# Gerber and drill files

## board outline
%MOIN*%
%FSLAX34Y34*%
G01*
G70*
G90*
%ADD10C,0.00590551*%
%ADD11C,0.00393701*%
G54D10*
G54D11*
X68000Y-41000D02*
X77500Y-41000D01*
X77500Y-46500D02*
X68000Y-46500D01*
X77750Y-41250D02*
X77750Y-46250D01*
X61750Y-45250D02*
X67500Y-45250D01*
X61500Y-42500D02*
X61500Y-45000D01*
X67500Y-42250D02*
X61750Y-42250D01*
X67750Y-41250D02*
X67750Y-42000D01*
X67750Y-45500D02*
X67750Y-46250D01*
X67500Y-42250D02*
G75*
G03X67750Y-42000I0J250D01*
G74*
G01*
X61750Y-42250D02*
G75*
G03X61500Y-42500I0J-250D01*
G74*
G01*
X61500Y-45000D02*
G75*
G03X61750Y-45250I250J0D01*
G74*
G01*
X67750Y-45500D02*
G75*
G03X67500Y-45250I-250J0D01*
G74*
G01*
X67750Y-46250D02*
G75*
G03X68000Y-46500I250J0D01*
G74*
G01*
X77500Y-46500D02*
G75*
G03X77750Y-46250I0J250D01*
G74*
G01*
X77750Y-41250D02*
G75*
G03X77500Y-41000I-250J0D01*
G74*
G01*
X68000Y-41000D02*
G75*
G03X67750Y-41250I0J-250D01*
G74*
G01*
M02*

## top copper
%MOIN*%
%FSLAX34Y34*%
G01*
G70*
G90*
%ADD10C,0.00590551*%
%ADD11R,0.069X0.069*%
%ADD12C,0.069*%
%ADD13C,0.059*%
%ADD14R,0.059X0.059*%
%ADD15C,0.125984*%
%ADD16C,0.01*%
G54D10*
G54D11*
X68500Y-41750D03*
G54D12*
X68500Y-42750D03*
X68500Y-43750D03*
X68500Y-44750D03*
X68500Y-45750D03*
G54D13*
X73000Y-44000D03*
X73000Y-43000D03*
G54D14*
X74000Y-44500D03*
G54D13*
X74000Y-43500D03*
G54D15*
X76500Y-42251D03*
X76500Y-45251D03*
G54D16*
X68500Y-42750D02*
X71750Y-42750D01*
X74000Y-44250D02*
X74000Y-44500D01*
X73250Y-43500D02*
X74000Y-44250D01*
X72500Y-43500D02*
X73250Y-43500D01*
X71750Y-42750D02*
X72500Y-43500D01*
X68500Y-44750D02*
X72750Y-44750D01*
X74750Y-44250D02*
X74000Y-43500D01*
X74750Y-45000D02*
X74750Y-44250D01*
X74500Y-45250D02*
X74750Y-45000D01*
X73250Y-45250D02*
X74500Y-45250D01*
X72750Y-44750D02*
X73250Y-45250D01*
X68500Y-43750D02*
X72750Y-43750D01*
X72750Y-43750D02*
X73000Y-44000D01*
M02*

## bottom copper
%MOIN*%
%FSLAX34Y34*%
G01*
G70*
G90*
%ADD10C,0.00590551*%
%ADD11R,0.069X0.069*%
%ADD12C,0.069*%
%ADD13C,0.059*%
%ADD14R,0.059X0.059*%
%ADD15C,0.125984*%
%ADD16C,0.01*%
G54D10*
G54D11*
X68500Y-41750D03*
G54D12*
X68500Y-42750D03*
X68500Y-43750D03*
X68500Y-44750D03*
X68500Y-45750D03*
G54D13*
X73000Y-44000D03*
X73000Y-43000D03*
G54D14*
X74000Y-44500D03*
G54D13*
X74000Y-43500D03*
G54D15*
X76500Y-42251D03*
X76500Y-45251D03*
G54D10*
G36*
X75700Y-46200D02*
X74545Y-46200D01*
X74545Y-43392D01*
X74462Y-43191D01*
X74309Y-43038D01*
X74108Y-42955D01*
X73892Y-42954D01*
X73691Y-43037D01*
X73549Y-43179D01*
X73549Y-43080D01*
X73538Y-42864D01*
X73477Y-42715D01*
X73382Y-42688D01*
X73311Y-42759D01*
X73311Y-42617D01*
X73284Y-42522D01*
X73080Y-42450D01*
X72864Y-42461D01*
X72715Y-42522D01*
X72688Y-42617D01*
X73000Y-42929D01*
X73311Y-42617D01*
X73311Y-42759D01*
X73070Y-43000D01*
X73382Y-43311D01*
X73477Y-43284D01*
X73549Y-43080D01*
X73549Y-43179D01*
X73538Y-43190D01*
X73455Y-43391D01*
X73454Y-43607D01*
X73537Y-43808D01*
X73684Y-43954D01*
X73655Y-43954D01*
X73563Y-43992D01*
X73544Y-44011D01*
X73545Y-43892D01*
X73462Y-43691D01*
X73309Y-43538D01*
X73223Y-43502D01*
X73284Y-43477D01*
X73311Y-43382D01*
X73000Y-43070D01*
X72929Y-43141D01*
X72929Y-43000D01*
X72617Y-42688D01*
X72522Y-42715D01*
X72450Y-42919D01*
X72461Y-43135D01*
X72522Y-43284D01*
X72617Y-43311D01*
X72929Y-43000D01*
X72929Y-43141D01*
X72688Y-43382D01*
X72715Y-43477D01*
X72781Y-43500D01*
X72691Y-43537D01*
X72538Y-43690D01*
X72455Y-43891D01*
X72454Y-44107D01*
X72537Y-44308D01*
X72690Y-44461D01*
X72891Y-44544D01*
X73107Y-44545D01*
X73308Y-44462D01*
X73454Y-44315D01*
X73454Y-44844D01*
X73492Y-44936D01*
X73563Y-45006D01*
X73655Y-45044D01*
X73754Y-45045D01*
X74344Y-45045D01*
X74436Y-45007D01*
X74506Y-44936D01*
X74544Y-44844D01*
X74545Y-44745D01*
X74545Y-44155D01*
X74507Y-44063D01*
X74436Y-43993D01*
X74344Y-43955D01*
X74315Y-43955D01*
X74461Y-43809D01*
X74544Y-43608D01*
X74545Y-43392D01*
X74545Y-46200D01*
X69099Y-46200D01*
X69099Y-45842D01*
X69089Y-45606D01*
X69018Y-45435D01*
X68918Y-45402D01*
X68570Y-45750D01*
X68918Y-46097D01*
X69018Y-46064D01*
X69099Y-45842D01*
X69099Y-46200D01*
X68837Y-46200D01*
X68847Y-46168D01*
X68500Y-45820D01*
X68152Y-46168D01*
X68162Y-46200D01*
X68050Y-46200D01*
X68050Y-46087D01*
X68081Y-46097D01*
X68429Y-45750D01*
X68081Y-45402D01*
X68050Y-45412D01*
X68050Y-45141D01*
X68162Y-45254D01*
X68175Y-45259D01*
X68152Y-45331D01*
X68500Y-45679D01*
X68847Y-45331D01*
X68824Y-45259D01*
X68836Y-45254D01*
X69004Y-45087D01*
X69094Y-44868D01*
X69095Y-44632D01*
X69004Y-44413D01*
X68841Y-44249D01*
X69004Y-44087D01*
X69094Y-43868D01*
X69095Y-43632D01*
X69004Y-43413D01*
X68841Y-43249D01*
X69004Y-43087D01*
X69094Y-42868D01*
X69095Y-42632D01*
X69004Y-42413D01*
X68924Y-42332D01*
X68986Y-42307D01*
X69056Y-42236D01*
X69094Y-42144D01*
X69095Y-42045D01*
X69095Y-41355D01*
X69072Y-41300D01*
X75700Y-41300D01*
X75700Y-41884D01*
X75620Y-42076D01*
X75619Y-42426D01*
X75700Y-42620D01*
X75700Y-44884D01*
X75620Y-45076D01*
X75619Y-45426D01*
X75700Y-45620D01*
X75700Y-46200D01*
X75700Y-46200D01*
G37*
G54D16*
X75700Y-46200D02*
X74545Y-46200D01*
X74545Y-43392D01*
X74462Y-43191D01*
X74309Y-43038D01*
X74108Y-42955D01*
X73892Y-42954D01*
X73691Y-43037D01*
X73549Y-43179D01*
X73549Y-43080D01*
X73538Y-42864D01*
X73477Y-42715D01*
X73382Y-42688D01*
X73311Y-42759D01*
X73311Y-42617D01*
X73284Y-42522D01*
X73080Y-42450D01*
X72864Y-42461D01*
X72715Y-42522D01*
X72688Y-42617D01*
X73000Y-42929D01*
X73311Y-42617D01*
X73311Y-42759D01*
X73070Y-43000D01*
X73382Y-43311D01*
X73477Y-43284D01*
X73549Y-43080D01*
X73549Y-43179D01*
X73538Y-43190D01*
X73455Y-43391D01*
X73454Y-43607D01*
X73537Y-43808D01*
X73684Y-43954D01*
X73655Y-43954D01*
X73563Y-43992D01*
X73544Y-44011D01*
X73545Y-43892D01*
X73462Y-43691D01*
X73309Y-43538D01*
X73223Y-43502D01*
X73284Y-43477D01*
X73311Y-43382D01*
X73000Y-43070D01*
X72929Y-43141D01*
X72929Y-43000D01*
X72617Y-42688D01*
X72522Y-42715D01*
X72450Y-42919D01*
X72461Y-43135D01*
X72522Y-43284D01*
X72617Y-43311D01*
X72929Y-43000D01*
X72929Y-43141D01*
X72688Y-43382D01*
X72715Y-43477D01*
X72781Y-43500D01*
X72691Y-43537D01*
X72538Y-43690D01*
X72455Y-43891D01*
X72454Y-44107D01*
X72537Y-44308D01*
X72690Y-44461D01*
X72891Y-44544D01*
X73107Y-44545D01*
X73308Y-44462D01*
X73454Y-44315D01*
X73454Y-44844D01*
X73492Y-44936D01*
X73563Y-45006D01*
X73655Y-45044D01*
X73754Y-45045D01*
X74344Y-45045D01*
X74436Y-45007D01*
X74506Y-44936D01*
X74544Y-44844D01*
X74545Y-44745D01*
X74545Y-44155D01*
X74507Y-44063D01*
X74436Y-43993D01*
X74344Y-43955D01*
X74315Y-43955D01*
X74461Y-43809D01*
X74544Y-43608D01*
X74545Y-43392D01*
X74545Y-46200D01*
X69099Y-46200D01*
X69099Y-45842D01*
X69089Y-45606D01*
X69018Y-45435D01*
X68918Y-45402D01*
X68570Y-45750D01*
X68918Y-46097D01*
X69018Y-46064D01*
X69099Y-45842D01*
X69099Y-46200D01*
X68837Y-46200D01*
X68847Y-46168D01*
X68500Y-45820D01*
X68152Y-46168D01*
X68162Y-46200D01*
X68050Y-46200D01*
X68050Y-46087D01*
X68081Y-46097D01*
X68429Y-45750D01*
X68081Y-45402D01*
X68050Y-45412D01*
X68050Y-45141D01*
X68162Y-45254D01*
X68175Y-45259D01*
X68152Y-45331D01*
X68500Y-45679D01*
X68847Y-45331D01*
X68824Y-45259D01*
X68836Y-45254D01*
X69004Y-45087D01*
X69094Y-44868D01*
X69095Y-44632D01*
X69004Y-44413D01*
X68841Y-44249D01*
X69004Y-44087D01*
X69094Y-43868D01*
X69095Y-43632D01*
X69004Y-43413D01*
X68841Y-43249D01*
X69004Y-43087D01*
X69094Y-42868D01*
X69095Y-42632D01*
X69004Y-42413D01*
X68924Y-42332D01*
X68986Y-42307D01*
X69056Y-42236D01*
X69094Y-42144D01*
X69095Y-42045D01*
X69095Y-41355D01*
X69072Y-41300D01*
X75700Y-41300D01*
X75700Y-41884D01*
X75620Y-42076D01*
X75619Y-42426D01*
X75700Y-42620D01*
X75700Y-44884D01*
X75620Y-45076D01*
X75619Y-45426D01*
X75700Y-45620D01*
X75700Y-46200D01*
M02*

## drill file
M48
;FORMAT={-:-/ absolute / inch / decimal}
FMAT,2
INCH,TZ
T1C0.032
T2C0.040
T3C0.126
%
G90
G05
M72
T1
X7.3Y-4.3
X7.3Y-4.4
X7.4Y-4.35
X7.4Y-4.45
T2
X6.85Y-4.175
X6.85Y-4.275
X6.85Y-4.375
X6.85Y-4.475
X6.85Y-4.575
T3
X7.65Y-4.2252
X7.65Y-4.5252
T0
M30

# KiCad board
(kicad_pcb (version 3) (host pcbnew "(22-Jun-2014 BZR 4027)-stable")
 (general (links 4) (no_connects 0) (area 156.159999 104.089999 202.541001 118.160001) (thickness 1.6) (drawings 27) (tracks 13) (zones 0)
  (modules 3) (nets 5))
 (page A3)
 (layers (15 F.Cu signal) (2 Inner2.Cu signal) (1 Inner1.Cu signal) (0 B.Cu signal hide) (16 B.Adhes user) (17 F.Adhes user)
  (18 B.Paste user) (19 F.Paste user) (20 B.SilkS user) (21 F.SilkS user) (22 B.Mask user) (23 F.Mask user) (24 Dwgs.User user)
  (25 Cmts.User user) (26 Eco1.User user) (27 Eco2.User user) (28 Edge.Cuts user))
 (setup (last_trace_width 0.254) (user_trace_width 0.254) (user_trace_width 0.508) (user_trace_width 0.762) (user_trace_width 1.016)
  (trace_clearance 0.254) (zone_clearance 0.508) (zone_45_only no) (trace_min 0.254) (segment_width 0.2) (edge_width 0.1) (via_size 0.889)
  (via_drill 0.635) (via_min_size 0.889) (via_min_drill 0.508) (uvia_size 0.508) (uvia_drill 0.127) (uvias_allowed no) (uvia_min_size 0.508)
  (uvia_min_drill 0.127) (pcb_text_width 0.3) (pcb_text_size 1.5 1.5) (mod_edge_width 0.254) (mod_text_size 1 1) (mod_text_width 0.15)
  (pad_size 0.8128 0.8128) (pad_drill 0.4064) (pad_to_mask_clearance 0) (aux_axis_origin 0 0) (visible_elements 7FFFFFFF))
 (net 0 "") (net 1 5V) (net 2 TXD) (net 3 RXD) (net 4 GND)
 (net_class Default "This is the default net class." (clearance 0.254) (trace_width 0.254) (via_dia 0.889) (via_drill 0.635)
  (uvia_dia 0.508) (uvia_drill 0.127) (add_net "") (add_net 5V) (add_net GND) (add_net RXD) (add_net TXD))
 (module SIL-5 (layer F.Cu) (at 173.99 108.585 270)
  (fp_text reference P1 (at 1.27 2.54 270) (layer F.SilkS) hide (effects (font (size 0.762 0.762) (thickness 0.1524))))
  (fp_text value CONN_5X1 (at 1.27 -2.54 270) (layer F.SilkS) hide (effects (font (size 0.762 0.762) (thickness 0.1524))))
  (pad 1 thru_hole rect (at -2.54 0 270) (size 1.7526 1.7526) (drill 1.016) (layers *.Cu *.Mask F.SilkS))
  (pad 2 thru_hole circle (at 0 0 270) (size 1.7526 1.7526) (drill 1.016) (layers *.Cu *.Mask F.SilkS) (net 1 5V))
  (pad 3 thru_hole circle (at 2.54 0 270) (size 1.7526 1.7526) (drill 1.016) (layers *.Cu *.Mask F.SilkS) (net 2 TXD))
  (pad 4 thru_hole circle (at 5.08 0 270) (size 1.7526 1.7526) (drill 1.016) (layers *.Cu *.Mask F.SilkS) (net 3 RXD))
  (pad 5 thru_hole circle (at 7.62 0 270) (size 1.7526 1.7526) (drill 1.016) (layers *.Cu *.Mask F.SilkS) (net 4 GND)))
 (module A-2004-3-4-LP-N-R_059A (layer F.Cu) (at 187.96 113.03 90)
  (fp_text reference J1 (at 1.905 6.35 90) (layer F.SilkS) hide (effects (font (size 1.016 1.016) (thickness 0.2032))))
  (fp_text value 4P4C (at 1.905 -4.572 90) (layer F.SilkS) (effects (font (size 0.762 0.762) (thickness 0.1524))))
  (pad 2 thru_hole circle (at 1.27 -2.54 90) (size 1.4986 1.4986) (drill 0.8128) (layers *.Cu *.Mask F.SilkS) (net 2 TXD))
  (pad 4 thru_hole circle (at 3.81 -2.54 90) (size 1.4986 1.4986) (drill 0.8128) (layers *.Cu *.Mask F.SilkS) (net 4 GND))
  (pad 1 thru_hole rect (at 0 0 90) (size 1.4986 1.4986) (drill 0.8128) (layers *.Cu *.Mask F.SilkS) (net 1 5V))
  (pad 3 thru_hole circle (at 2.54 0 90) (size 1.4986 1.4986) (drill 0.8128) (layers *.Cu *.Mask F.SilkS) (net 3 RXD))
  (pad "" thru_hole circle (at 5.71 6.35 90) (size 3.2 3.2) (drill 3.2) (layers *.Cu *.Mask F.SilkS))
  (pad "" thru_hole circle (at -1.91 6.35 90) (size 3.2 3.2) (drill 3.2) (layers *.Cu *.Mask F.SilkS)))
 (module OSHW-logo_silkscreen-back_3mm (layer F.Cu) (at 169.545 111.125)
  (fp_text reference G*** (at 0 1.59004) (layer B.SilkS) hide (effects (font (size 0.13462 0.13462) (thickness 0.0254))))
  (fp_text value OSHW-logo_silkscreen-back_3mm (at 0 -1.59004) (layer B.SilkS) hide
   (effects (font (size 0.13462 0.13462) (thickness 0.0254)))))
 (gr_line (start 172.72 104.14) (end 196.85 104.14) (angle 90) (layer Edge.Cuts) (width 0.1))
 (gr_line (start 196.85 118.11) (end 172.72 118.11) (angle 90) (layer Edge.Cuts) (width 0.1))
 (gr_line (start 197.485 104.775) (end 197.485 117.475) (angle 90) (layer Edge.Cuts) (width 0.1))
 (gr_line (start 156.845 114.935) (end 171.45 114.935) (angle 90) (layer Edge.Cuts) (width 0.1))
 (gr_line (start 156.21 107.95) (end 156.21 114.3) (angle 90) (layer Edge.Cuts) (width 0.1))
 (gr_line (start 171.45 107.315) (end 156.845 107.315) (angle 90) (layer Edge.Cuts) (width 0.1))
 (gr_line (start 172.085 104.775) (end 172.085 106.68) (angle 90) (layer Edge.Cuts) (width 0.1))
 (gr_line (start 172.085 115.57) (end 172.085 117.475) (angle 90) (layer Edge.Cuts) (width 0.1))
 (gr_arc (start 171.45 106.68) (end 172.085 106.68) (angle 90) (layer Edge.Cuts) (width 0.1))
 (gr_arc (start 156.845 107.95) (end 156.21 107.95) (angle 90) (layer Edge.Cuts) (width 0.1))
 (gr_arc (start 156.845 114.3) (end 156.845 114.935) (angle 90) (layer Edge.Cuts) (width 0.1))
 (gr_arc (start 171.45 115.57) (end 171.45 114.935) (angle 90) (layer Edge.Cuts) (width 0.1))
 (gr_arc (start 172.72 117.475) (end 172.72 118.11) (angle 90) (layer Edge.Cuts) (width 0.1))
 (gr_arc (start 196.85 117.475) (end 197.485 117.475) (angle 90) (layer Edge.Cuts) (width 0.1))
 (gr_arc (start 196.85 104.775) (end 196.85 104.14) (angle 90) (layer Edge.Cuts) (width 0.1))
 (gr_arc (start 172.72 104.775) (end 172.085 104.775) (angle 90) (layer Edge.Cuts) (width 0.1))
 (segment (start 173.99 108.585) (end 182.245 108.585) (width 0.254) (layer F.Cu) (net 1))
 (segment (start 187.96 112.395) (end 187.96 113.03) (width 0.254) (layer F.Cu) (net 1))
 (segment (start 186.055 110.49) (end 187.96 112.395) (width 0.254) (layer F.Cu) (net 1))
 (segment (start 184.15 110.49) (end 186.055 110.49) (width 0.254) (layer F.Cu) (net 1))
 (segment (start 182.245 108.585) (end 184.15 110.49) (width 0.254) (layer F.Cu) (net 1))
 (segment (start 173.99 113.665) (end 184.785 113.665) (width 0.254) (layer F.Cu) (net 3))
 (segment (start 189.865 112.395) (end 187.96 110.49) (width 0.254) (layer F.Cu) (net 3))
 (segment (start 189.865 114.3) (end 189.865 112.395) (width 0.254) (layer F.Cu) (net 3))
 (segment (start 189.23 114.935) (end 189.865 114.3) (width 0.254) (layer F.Cu) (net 3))
 (segment (start 186.055 114.935) (end 189.23 114.935) (width 0.254) (layer F.Cu) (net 3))
 (segment (start 184.785 113.665) (end 186.055 114.935) (width 0.254) (layer F.Cu) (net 3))
 (segment (start 173.99 111.125) (end 184.785 111.125) (width 0.254) (layer F.Cu) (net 2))
 (segment (start 184.785 111.125) (end 185.42 111.76) (width 0.254) (layer F.Cu) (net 2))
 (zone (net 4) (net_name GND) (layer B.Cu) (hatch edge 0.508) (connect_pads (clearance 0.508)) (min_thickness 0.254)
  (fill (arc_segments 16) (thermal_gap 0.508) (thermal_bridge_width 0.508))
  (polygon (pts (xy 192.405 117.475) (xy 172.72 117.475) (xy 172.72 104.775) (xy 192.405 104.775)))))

